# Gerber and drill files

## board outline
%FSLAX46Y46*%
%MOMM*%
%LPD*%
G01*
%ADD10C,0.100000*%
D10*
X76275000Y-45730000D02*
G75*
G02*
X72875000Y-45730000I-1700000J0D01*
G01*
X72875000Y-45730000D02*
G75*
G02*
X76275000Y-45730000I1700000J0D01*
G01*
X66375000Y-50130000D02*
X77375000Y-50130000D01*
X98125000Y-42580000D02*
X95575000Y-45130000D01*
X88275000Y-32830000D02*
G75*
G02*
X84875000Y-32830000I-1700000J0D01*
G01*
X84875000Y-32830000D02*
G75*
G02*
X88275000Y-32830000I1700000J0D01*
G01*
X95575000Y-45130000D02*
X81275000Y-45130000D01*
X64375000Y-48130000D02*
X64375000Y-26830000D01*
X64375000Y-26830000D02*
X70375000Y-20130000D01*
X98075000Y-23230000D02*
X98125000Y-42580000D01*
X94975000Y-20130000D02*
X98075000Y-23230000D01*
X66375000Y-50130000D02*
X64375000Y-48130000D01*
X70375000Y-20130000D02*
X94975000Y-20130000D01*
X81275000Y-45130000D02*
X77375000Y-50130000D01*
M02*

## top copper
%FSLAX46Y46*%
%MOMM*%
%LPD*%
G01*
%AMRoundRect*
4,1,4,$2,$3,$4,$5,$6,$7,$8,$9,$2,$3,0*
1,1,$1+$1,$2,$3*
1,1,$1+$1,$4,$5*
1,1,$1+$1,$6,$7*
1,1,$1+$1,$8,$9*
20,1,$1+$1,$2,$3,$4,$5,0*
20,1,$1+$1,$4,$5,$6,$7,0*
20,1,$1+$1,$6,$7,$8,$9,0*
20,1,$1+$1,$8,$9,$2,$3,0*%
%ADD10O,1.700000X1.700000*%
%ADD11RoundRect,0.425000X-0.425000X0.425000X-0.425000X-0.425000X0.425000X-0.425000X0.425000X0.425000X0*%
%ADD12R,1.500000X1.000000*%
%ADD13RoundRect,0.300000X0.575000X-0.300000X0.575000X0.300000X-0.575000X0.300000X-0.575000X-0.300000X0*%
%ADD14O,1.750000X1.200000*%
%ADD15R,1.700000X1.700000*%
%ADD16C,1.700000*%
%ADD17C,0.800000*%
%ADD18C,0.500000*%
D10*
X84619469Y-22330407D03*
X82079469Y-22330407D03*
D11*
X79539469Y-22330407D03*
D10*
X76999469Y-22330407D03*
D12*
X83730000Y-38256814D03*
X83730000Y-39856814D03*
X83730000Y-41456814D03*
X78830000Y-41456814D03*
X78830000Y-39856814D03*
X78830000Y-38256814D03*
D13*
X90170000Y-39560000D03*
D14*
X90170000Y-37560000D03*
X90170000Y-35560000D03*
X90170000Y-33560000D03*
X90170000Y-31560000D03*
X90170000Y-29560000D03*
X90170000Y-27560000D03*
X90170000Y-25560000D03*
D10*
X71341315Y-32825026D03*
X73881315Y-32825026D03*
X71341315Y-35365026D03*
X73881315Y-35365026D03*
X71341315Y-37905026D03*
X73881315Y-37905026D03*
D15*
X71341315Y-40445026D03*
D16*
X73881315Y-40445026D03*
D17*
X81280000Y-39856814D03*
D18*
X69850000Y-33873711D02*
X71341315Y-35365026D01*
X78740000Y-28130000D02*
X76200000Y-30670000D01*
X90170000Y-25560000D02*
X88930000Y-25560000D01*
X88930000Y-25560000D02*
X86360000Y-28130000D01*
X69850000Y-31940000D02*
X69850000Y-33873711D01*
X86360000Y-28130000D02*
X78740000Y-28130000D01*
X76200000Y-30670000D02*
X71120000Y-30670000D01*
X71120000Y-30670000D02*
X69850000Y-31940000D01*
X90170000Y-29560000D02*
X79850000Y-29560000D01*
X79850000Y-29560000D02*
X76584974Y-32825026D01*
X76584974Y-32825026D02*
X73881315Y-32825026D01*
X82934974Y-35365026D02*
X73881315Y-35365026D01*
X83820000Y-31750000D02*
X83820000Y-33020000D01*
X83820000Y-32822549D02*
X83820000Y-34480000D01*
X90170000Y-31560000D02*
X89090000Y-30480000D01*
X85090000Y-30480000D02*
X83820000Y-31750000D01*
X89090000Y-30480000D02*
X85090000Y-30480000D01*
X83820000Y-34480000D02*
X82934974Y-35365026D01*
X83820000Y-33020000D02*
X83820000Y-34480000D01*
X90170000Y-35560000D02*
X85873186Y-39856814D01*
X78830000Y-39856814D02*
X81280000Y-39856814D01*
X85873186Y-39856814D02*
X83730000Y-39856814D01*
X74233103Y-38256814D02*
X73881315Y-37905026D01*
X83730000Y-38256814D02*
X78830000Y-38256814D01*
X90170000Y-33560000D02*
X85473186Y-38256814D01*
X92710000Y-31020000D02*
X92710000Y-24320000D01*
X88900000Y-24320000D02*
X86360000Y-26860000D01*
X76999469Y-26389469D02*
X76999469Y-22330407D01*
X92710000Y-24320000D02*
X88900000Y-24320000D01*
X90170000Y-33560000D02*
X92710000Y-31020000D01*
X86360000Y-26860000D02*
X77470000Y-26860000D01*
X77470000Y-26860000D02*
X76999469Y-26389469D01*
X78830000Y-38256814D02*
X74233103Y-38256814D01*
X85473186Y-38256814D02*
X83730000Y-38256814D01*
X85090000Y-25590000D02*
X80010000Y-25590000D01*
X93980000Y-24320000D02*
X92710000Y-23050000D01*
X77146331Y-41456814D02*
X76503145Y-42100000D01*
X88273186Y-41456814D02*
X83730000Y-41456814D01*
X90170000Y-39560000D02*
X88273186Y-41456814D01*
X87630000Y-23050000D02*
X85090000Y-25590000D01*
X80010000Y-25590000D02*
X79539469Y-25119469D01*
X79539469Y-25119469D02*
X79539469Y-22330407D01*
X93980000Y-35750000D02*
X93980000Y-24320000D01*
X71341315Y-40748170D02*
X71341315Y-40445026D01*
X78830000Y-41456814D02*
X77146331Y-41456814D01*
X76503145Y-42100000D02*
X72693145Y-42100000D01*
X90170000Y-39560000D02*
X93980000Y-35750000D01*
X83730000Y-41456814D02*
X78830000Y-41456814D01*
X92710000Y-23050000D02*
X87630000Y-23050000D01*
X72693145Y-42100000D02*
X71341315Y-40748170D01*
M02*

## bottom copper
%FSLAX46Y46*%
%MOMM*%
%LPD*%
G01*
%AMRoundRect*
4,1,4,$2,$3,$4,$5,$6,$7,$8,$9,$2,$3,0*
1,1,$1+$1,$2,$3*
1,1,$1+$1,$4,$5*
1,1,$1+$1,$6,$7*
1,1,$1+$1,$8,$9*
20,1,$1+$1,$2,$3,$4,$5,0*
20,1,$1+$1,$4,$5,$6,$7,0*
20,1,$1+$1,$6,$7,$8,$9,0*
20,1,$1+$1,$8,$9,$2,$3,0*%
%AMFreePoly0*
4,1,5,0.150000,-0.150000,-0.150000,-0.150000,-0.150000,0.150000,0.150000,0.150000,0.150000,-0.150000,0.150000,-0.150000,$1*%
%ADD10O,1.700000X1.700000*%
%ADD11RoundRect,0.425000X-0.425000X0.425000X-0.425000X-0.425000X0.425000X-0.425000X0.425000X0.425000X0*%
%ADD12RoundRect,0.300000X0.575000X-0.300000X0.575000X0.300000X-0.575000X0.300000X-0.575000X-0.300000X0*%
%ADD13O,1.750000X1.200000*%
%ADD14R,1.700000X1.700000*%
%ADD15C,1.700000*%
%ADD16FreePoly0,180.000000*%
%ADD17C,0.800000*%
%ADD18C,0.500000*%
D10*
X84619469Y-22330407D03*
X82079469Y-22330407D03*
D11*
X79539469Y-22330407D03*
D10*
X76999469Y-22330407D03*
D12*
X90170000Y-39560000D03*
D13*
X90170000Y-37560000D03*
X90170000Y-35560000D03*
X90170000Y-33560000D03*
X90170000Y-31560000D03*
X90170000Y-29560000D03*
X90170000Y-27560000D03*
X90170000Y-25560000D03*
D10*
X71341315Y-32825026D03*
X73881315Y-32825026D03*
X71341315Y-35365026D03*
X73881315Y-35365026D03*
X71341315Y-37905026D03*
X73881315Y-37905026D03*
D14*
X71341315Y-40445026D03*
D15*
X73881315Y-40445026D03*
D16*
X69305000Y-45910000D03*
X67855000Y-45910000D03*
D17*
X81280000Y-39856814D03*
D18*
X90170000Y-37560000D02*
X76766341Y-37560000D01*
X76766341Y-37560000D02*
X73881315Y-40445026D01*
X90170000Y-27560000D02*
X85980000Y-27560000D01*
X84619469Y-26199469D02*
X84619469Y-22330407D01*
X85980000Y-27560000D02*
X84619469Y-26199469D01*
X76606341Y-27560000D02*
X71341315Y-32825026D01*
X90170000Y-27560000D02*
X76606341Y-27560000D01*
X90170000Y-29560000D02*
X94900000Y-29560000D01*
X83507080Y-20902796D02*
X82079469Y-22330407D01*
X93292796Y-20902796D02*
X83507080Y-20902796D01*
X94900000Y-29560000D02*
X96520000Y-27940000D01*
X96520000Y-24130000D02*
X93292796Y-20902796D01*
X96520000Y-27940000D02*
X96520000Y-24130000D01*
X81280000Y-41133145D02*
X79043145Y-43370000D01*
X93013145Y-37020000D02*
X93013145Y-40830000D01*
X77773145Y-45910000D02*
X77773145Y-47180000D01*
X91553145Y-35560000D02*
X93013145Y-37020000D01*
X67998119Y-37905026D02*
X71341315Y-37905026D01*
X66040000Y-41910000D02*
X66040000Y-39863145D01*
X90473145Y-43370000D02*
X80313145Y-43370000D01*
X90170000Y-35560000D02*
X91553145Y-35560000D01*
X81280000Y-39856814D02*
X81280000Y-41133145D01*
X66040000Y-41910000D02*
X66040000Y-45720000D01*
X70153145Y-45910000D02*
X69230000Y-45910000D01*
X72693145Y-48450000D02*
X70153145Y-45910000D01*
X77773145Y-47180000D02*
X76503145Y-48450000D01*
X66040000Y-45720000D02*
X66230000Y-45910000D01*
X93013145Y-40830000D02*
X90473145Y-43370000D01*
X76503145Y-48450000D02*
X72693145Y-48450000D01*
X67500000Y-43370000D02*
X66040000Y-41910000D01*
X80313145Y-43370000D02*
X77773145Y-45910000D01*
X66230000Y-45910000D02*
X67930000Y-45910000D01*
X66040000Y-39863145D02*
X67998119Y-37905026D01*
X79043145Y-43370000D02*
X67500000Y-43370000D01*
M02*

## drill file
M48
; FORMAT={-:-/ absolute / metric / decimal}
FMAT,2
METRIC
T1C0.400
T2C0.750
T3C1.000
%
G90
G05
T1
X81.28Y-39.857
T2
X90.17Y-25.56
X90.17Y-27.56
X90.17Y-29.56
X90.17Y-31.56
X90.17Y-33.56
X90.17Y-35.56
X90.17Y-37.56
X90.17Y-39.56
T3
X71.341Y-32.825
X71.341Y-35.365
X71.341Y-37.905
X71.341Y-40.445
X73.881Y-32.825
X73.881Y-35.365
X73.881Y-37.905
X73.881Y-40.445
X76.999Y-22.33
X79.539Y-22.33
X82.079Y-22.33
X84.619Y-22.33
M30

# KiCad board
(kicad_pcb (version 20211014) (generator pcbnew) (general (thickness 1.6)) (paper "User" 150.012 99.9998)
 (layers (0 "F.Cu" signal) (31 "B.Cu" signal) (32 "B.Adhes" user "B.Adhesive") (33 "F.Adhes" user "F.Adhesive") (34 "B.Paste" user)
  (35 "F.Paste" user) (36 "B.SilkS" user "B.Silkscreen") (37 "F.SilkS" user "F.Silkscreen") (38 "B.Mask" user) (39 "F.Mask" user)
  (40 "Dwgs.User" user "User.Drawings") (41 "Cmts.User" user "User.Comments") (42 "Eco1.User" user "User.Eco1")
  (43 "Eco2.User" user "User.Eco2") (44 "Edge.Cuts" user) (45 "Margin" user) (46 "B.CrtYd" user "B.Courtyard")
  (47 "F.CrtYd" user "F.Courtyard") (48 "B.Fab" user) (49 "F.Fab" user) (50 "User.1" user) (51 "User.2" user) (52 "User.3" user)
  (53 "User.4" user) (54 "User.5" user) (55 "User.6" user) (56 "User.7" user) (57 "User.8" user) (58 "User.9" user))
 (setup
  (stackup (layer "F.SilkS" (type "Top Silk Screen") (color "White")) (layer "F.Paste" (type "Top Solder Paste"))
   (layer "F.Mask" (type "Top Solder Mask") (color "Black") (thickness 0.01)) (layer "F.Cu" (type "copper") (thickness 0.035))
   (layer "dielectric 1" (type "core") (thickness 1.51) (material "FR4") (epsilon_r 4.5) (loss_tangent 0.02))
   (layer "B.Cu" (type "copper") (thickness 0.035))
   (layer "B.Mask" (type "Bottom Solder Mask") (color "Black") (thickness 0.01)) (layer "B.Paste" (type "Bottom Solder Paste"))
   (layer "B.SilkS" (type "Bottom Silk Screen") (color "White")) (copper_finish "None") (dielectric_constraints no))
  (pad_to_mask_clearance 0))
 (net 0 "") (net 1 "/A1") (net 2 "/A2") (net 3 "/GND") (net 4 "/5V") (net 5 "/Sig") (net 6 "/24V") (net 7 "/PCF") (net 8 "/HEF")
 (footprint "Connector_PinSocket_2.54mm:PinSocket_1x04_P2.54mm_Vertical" (layer "F.Cu") (at 84.619469 22.330407 -90)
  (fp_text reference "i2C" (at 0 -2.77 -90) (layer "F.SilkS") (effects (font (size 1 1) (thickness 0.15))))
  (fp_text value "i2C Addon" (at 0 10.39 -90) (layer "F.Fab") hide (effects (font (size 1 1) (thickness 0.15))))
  (pad "1" thru_hole oval (at 0 0 270) (size 1.7 1.7) (drill 1) (layers *.Cu *.Mask) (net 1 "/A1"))
  (pad "2" thru_hole oval (at 0 2.54 270) (size 1.7 1.7) (drill 1) (layers *.Cu *.Mask) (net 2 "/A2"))
  (pad "3" thru_hole roundrect (at 0 5.08 270) (size 1.7 1.7) (drill 1) (layers *.Cu *.Mask) (roundrect_rratio 0.25) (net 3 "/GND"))
  (pad "4" thru_hole oval (at 0 7.62 270) (size 1.7 1.7) (drill 1) (layers *.Cu *.Mask) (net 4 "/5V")))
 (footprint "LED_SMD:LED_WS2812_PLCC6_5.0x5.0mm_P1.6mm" (layer "F.Cu") (at 81.28 39.856814)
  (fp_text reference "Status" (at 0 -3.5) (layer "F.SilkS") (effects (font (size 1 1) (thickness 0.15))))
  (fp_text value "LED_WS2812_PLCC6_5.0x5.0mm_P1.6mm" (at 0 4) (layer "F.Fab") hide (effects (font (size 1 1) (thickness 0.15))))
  (pad "1" smd rect (at 2.45 -1.6) (size 1.5 1) (layers "F.Cu" "F.Paste" "F.Mask") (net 4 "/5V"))
  (pad "2" smd rect (at 2.45 0) (size 1.5 1) (layers "F.Cu" "F.Paste" "F.Mask") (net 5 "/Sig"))
  (pad "3" smd rect (at 2.45 1.6) (size 1.5 1) (layers "F.Cu" "F.Paste" "F.Mask") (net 3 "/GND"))
  (pad "4" smd rect (at -2.45 1.6) (size 1.5 1) (layers "F.Cu" "F.Paste" "F.Mask") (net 3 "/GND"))
  (pad "5" smd rect (at -2.45 0) (size 1.5 1) (layers "F.Cu" "F.Paste" "F.Mask") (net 5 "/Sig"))
  (pad "6" smd rect (at -2.45 -1.6) (size 1.5 1) (layers "F.Cu" "F.Paste" "F.Mask") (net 4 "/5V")))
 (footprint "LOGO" (layer "F.Cu") (at 68.58 26.86)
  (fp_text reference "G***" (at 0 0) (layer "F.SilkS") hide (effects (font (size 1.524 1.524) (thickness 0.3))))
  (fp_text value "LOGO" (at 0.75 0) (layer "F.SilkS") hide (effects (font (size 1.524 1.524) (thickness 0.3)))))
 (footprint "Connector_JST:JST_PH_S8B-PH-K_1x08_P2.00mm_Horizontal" (layer "F.Cu") (at 90.17 39.56 90)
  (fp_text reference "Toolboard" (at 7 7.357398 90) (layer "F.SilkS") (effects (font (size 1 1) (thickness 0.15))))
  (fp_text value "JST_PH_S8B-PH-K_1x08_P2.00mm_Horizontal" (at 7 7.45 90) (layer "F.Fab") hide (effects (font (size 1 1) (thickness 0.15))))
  (pad "1" thru_hole roundrect (at 0 0 90) (size 1.2 1.75) (drill 0.75) (layers *.Cu *.Mask) (roundrect_rratio 0.25) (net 3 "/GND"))
  (pad "2" thru_hole oval (at 2 0 90) (size 1.2 1.75) (drill 0.75) (layers *.Cu *.Mask) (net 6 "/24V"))
  (pad "3" thru_hole oval (at 4 0 90) (size 1.2 1.75) (drill 0.75) (layers *.Cu *.Mask) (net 5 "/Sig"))
  (pad "4" thru_hole oval (at 6 0 90) (size 1.2 1.75) (drill 0.75) (layers *.Cu *.Mask) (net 4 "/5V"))
  (pad "5" thru_hole oval (at 8 0 90) (size 1.2 1.75) (drill 0.75) (layers *.Cu *.Mask) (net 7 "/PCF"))
  (pad "6" thru_hole oval (at 10 0 90) (size 1.2 1.75) (drill 0.75) (layers *.Cu *.Mask) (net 2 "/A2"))
  (pad "7" thru_hole oval (at 12 0 90) (size 1.2 1.75) (drill 0.75) (layers *.Cu *.Mask) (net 1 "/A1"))
  (pad "8" thru_hole oval (at 14 0 90) (size 1.2 1.75) (drill 0.75) (layers *.Cu *.Mask) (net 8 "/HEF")))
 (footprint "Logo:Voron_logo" (layer "F.Cu") (at 80.775 32.73)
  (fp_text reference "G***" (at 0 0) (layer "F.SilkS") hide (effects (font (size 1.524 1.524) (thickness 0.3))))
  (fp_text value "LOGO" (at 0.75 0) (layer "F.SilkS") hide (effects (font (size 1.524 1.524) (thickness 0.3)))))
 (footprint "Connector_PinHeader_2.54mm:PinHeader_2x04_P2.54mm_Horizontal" (layer "F.Cu") (at 63.261315 32.825026)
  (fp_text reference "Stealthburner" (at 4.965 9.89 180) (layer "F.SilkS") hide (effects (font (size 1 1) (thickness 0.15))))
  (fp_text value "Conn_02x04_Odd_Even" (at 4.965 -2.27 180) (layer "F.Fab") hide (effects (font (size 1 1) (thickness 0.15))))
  (pad "1" thru_hole oval (at 8.08 0 180) (size 1.7 1.7) (drill 1) (layers *.Cu *.Mask) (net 1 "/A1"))
  (pad "2" thru_hole oval (at 10.62 0 180) (size 1.7 1.7) (drill 1) (layers *.Cu *.Mask) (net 2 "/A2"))
  (pad "3" thru_hole oval (at 8.08 2.54 180) (size 1.7 1.7) (drill 1) (layers *.Cu *.Mask) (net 8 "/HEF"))
  (pad "4" thru_hole oval (at 10.62 2.54 180) (size 1.7 1.7) (drill 1) (layers *.Cu *.Mask) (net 7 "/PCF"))
  (pad "5" thru_hole oval (at 8.08 5.08 180) (size 1.7 1.7) (drill 1) (layers *.Cu *.Mask) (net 5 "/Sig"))
  (pad "6" thru_hole oval (at 10.62 5.08 180) (size 1.7 1.7) (drill 1) (layers *.Cu *.Mask) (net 4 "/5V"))
  (pad "7" thru_hole rect (at 8.08 7.62 180) (size 1.7 1.7) (drill 1) (layers *.Cu *.Mask) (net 3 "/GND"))
  (pad "8" thru_hole circle (at 10.62 7.62 180) (size 1.7 1.7) (drill 1) (layers *.Cu *.Mask) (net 6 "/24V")))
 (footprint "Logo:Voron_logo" (layer "B.Cu") (at 80.775 32.73 180)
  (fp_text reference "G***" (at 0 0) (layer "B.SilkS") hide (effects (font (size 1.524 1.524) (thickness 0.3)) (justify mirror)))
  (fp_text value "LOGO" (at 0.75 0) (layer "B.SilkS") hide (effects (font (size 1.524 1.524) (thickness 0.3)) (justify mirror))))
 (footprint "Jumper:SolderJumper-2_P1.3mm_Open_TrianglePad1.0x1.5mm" (layer "B.Cu") (at 68.58 45.91 180)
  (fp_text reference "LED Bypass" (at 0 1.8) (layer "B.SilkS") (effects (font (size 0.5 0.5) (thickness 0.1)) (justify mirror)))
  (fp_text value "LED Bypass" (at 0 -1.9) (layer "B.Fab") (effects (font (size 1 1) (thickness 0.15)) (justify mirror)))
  (pad "1" smd custom (at -0.725 0 180) (size 0.3 0.3) (layers "B.Cu" "B.Mask") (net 5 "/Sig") (zone_connect 2)
   (options (clearance outline) (anchor rect)) (primitives))
  (pad "2" smd custom (at 0.725 0 180) (size 0.3 0.3) (layers "B.Cu" "B.Mask") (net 5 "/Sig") (zone_connect 2)
   (options (clearance outline) (anchor rect)) (primitives)))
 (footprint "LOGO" (layer "B.Cu") (at 71.12 24.32 180)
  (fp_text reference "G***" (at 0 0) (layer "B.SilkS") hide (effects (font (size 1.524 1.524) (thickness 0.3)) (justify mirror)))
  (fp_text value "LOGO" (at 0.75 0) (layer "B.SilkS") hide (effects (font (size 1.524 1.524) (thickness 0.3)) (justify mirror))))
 (gr_circle (center 74.575 45.73) (end 76.275 45.73) (layer "Edge.Cuts") (width 0.1) (fill none))
 (gr_line (start 66.375 50.13) (end 77.375 50.13) (layer "Edge.Cuts") (width 0.1))
 (gr_line (start 98.125 42.58) (end 95.575 45.13) (layer "Edge.Cuts") (width 0.1))
 (gr_circle (center 86.575 32.83) (end 88.275 32.83) (layer "Edge.Cuts") (width 0.1) (fill none))
 (gr_line (start 95.575 45.13) (end 81.275 45.13) (layer "Edge.Cuts") (width 0.1))
 (gr_line (start 64.375 48.13) (end 64.375 26.83) (layer "Edge.Cuts") (width 0.1))
 (gr_line (start 64.375 26.83) (end 70.375 20.13) (layer "Edge.Cuts") (width 0.1))
 (gr_line (start 98.075 23.23) (end 98.125 42.58) (layer "Edge.Cuts") (width 0.1))
 (gr_line (start 94.975 20.13) (end 98.075 23.23) (layer "Edge.Cuts") (width 0.1))
 (gr_line (start 66.375 50.13) (end 64.375 48.13) (layer "Edge.Cuts") (width 0.1))
 (gr_line (start 70.375 20.13) (end 94.975 20.13) (layer "Edge.Cuts") (width 0.1))
 (gr_line (start 81.275 45.13) (end 77.375 50.13) (layer "Edge.Cuts") (width 0.1))
 (segment (start 90.17 37.56) (end 76.766341 37.56) (width 0.5) (layer "B.Cu") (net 6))
 (segment (start 76.766341 37.56) (end 73.881315 40.445026) (width 0.5) (layer "B.Cu") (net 6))
 (segment (start 69.85 33.873711) (end 71.341315 35.365026) (width 0.5) (layer "F.Cu") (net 8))
 (segment (start 78.74 28.13) (end 76.2 30.67) (width 0.5) (layer "F.Cu") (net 8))
 (segment (start 90.17 25.56) (end 88.93 25.56) (width 0.5) (layer "F.Cu") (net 8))
 (segment (start 88.93 25.56) (end 86.36 28.13) (width 0.5) (layer "F.Cu") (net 8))
 (segment (start 69.85 31.94) (end 69.85 33.873711) (width 0.5) (layer "F.Cu") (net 8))
 (segment (start 86.36 28.13) (end 78.74 28.13) (width 0.5) (layer "F.Cu") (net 8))
 (segment (start 76.2 30.67) (end 71.12 30.67) (width 0.5) (layer "F.Cu") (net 8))
 (segment (start 71.12 30.67) (end 69.85 31.94) (width 0.5) (layer "F.Cu") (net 8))
 (segment (start 90.17 27.56) (end 85.98 27.56) (width 0.5) (layer "B.Cu") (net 1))
 (segment (start 84.619469 26.199469) (end 84.619469 22.330407) (width 0.5) (layer "B.Cu") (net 1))
 (segment (start 85.98 27.56) (end 84.619469 26.199469) (width 0.5) (layer "B.Cu") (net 1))
 (segment (start 76.606341 27.56) (end 71.341315 32.825026) (width 0.5) (layer "B.Cu") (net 1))
 (segment (start 90.17 27.56) (end 76.606341 27.56) (width 0.5) (layer "B.Cu") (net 1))
 (segment (start 90.17 29.56) (end 79.85 29.56) (width 0.5) (layer "F.Cu") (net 2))
 (segment (start 79.85 29.56) (end 76.584974 32.825026) (width 0.5) (layer "F.Cu") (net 2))
 (segment (start 76.584974 32.825026) (end 73.881315 32.825026) (width 0.5) (layer "F.Cu") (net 2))
 (segment (start 90.17 29.56) (end 94.9 29.56) (width 0.5) (layer "B.Cu") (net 2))
 (segment (start 83.50708 20.902796) (end 82.079469 22.330407) (width 0.5) (layer "B.Cu") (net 2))
 (segment (start 93.292796 20.902796) (end 83.50708 20.902796) (width 0.5) (layer "B.Cu") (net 2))
 (segment (start 94.9 29.56) (end 96.52 27.94) (width 0.5) (layer "B.Cu") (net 2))
 (segment (start 96.52 24.13) (end 93.292796 20.902796) (width 0.5) (layer "B.Cu") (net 2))
 (segment (start 96.52 27.94) (end 96.52 24.13) (width 0.5) (layer "B.Cu") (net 2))
 (segment (start 82.934974 35.365026) (end 73.881315 35.365026) (width 0.5) (layer "F.Cu") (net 7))
 (segment (start 83.82 31.75) (end 83.82 33.02) (width 0.5) (layer "F.Cu") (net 7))
 (segment (start 83.82 32.822549) (end 83.82 34.48) (width 0.5) (layer "F.Cu") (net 7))
 (segment (start 90.17 31.56) (end 89.09 30.48) (width 0.5) (layer "F.Cu") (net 7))
 (segment (start 85.09 30.48) (end 83.82 31.75) (width 0.5) (layer "F.Cu") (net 7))
 (segment (start 89.09 30.48) (end 85.09 30.48) (width 0.5) (layer "F.Cu") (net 7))
 (segment (start 83.82 34.48) (end 82.934974 35.365026) (width 0.5) (layer "F.Cu") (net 7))
 (segment (start 83.82 33.02) (end 83.82 34.48) (width 0.5) (layer "F.Cu") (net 7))
 (segment (start 90.17 35.56) (end 85.873186 39.856814) (width 0.5) (layer "F.Cu") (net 5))
 (segment (start 78.83 39.856814) (end 81.28 39.856814) (width 0.5) (layer "F.Cu") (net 5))
 (segment (start 85.873186 39.856814) (end 83.73 39.856814) (width 0.5) (layer "F.Cu") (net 5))
 (via blind (at 81.28 39.856814) (size 0.8) (drill 0.4) (layers "F.Cu" "B.Cu") (free) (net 5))
 (segment (start 81.28 41.133145) (end 79.043145 43.37) (width 0.5) (layer "B.Cu") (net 5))
 (segment (start 93.013145 37.02) (end 93.013145 40.83) (width 0.5) (layer "B.Cu") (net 5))
 (segment (start 77.773145 45.91) (end 77.773145 47.18) (width 0.5) (layer "B.Cu") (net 5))
 (segment (start 91.553145 35.56) (end 93.013145 37.02) (width 0.5) (layer "B.Cu") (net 5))
 (segment (start 67.998119 37.905026) (end 71.341315 37.905026) (width 0.5) (layer "B.Cu") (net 5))
 (segment (start 66.04 41.91) (end 66.04 39.863145) (width 0.5) (layer "B.Cu") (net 5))
 (segment (start 90.473145 43.37) (end 80.313145 43.37) (width 0.5) (layer "B.Cu") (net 5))
 (segment (start 90.17 35.56) (end 91.553145 35.56) (width 0.5) (layer "B.Cu") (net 5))
 (segment (start 81.28 39.856814) (end 81.28 41.133145) (width 0.5) (layer "B.Cu") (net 5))
 (segment (start 66.04 41.91) (end 66.04 45.72) (width 0.5) (layer "B.Cu") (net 5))
 (segment (start 70.153145 45.91) (end 69.23 45.91) (width 0.5) (layer "B.Cu") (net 5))
 (segment (start 72.693145 48.45) (end 70.153145 45.91) (width 0.5) (layer "B.Cu") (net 5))
 (segment (start 77.773145 47.18) (end 76.503145 48.45) (width 0.5) (layer "B.Cu") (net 5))
 (segment (start 66.04 45.72) (end 66.23 45.91) (width 0.5) (layer "B.Cu") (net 5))
 (segment (start 93.013145 40.83) (end 90.473145 43.37) (width 0.5) (layer "B.Cu") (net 5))
 (segment (start 76.503145 48.45) (end 72.693145 48.45) (width 0.5) (layer "B.Cu") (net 5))
 (segment (start 67.5 43.37) (end 66.04 41.91) (width 0.5) (layer "B.Cu") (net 5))
 (segment (start 80.313145 43.37) (end 77.773145 45.91) (width 0.5) (layer "B.Cu") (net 5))
 (segment (start 66.23 45.91) (end 67.93 45.91) (width 0.5) (layer "B.Cu") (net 5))
 (segment (start 66.04 39.863145) (end 67.998119 37.905026) (width 0.5) (layer "B.Cu") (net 5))
 (segment (start 79.043145 43.37) (end 67.5 43.37) (width 0.5) (layer "B.Cu") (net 5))
 (segment (start 74.233103 38.256814) (end 73.881315 37.905026) (width 0.5) (layer "F.Cu") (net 4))
 (segment (start 83.73 38.256814) (end 78.83 38.256814) (width 0.5) (layer "F.Cu") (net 4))
 (segment (start 90.17 33.56) (end 85.473186 38.256814) (width 0.5) (layer "F.Cu") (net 4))
 (segment (start 92.71 31.02) (end 92.71 24.32) (width 0.5) (layer "F.Cu") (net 4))
 (segment (start 88.9 24.32) (end 86.36 26.86) (width 0.5) (layer "F.Cu") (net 4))
 (segment (start 76.999469 26.389469) (end 76.999469 22.330407) (width 0.5) (layer "F.Cu") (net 4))
 (segment (start 92.71 24.32) (end 88.9 24.32) (width 0.5) (layer "F.Cu") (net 4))
 (segment (start 90.17 33.56) (end 92.71 31.02) (width 0.5) (layer "F.Cu") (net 4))
 (segment (start 86.36 26.86) (end 77.47 26.86) (width 0.5) (layer "F.Cu") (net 4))
 (segment (start 77.47 26.86) (end 76.999469 26.389469) (width 0.5) (layer "F.Cu") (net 4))
 (segment (start 78.83 38.256814) (end 74.233103 38.256814) (width 0.5) (layer "F.Cu") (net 4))
 (segment (start 85.473186 38.256814) (end 83.73 38.256814) (width 0.5) (layer "F.Cu") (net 4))
 (segment (start 85.09 25.59) (end 80.01 25.59) (width 0.5) (layer "F.Cu") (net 3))
 (segment (start 93.98 24.32) (end 92.71 23.05) (width 0.5) (layer "F.Cu") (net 3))
 (segment (start 77.146331 41.456814) (end 76.503145 42.1) (width 0.5) (layer "F.Cu") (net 3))
 (segment (start 88.273186 41.456814) (end 83.73 41.456814) (width 0.5) (layer "F.Cu") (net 3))
 (segment (start 90.17 39.56) (end 88.273186 41.456814) (width 0.5) (layer "F.Cu") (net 3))
 (segment (start 87.63 23.05) (end 85.09 25.59) (width 0.5) (layer "F.Cu") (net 3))
 (segment (start 80.01 25.59) (end 79.539469 25.119469) (width 0.5) (layer "F.Cu") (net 3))
 (segment (start 79.539469 25.119469) (end 79.539469 22.330407) (width 0.5) (layer "F.Cu") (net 3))
 (segment (start 93.98 35.75) (end 93.98 24.32) (width 0.5) (layer "F.Cu") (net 3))
 (segment (start 71.341315 40.74817) (end 71.341315 40.445026) (width 0.5) (layer "F.Cu") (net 3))
 (segment (start 78.83 41.456814) (end 77.146331 41.456814) (width 0.5) (layer "F.Cu") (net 3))
 (segment (start 76.503145 42.1) (end 72.693145 42.1) (width 0.5) (layer "F.Cu") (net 3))
 (segment (start 90.17 39.56) (end 93.98 35.75) (width 0.5) (layer "F.Cu") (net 3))
 (segment (start 83.73 41.456814) (end 78.83 41.456814) (width 0.5) (layer "F.Cu") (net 3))
 (segment (start 92.71 23.05) (end 87.63 23.05) (width 0.5) (layer "F.Cu") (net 3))
 (segment (start 72.693145 42.1) (end 71.341315 40.74817) (width 0.5) (layer "F.Cu") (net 3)))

